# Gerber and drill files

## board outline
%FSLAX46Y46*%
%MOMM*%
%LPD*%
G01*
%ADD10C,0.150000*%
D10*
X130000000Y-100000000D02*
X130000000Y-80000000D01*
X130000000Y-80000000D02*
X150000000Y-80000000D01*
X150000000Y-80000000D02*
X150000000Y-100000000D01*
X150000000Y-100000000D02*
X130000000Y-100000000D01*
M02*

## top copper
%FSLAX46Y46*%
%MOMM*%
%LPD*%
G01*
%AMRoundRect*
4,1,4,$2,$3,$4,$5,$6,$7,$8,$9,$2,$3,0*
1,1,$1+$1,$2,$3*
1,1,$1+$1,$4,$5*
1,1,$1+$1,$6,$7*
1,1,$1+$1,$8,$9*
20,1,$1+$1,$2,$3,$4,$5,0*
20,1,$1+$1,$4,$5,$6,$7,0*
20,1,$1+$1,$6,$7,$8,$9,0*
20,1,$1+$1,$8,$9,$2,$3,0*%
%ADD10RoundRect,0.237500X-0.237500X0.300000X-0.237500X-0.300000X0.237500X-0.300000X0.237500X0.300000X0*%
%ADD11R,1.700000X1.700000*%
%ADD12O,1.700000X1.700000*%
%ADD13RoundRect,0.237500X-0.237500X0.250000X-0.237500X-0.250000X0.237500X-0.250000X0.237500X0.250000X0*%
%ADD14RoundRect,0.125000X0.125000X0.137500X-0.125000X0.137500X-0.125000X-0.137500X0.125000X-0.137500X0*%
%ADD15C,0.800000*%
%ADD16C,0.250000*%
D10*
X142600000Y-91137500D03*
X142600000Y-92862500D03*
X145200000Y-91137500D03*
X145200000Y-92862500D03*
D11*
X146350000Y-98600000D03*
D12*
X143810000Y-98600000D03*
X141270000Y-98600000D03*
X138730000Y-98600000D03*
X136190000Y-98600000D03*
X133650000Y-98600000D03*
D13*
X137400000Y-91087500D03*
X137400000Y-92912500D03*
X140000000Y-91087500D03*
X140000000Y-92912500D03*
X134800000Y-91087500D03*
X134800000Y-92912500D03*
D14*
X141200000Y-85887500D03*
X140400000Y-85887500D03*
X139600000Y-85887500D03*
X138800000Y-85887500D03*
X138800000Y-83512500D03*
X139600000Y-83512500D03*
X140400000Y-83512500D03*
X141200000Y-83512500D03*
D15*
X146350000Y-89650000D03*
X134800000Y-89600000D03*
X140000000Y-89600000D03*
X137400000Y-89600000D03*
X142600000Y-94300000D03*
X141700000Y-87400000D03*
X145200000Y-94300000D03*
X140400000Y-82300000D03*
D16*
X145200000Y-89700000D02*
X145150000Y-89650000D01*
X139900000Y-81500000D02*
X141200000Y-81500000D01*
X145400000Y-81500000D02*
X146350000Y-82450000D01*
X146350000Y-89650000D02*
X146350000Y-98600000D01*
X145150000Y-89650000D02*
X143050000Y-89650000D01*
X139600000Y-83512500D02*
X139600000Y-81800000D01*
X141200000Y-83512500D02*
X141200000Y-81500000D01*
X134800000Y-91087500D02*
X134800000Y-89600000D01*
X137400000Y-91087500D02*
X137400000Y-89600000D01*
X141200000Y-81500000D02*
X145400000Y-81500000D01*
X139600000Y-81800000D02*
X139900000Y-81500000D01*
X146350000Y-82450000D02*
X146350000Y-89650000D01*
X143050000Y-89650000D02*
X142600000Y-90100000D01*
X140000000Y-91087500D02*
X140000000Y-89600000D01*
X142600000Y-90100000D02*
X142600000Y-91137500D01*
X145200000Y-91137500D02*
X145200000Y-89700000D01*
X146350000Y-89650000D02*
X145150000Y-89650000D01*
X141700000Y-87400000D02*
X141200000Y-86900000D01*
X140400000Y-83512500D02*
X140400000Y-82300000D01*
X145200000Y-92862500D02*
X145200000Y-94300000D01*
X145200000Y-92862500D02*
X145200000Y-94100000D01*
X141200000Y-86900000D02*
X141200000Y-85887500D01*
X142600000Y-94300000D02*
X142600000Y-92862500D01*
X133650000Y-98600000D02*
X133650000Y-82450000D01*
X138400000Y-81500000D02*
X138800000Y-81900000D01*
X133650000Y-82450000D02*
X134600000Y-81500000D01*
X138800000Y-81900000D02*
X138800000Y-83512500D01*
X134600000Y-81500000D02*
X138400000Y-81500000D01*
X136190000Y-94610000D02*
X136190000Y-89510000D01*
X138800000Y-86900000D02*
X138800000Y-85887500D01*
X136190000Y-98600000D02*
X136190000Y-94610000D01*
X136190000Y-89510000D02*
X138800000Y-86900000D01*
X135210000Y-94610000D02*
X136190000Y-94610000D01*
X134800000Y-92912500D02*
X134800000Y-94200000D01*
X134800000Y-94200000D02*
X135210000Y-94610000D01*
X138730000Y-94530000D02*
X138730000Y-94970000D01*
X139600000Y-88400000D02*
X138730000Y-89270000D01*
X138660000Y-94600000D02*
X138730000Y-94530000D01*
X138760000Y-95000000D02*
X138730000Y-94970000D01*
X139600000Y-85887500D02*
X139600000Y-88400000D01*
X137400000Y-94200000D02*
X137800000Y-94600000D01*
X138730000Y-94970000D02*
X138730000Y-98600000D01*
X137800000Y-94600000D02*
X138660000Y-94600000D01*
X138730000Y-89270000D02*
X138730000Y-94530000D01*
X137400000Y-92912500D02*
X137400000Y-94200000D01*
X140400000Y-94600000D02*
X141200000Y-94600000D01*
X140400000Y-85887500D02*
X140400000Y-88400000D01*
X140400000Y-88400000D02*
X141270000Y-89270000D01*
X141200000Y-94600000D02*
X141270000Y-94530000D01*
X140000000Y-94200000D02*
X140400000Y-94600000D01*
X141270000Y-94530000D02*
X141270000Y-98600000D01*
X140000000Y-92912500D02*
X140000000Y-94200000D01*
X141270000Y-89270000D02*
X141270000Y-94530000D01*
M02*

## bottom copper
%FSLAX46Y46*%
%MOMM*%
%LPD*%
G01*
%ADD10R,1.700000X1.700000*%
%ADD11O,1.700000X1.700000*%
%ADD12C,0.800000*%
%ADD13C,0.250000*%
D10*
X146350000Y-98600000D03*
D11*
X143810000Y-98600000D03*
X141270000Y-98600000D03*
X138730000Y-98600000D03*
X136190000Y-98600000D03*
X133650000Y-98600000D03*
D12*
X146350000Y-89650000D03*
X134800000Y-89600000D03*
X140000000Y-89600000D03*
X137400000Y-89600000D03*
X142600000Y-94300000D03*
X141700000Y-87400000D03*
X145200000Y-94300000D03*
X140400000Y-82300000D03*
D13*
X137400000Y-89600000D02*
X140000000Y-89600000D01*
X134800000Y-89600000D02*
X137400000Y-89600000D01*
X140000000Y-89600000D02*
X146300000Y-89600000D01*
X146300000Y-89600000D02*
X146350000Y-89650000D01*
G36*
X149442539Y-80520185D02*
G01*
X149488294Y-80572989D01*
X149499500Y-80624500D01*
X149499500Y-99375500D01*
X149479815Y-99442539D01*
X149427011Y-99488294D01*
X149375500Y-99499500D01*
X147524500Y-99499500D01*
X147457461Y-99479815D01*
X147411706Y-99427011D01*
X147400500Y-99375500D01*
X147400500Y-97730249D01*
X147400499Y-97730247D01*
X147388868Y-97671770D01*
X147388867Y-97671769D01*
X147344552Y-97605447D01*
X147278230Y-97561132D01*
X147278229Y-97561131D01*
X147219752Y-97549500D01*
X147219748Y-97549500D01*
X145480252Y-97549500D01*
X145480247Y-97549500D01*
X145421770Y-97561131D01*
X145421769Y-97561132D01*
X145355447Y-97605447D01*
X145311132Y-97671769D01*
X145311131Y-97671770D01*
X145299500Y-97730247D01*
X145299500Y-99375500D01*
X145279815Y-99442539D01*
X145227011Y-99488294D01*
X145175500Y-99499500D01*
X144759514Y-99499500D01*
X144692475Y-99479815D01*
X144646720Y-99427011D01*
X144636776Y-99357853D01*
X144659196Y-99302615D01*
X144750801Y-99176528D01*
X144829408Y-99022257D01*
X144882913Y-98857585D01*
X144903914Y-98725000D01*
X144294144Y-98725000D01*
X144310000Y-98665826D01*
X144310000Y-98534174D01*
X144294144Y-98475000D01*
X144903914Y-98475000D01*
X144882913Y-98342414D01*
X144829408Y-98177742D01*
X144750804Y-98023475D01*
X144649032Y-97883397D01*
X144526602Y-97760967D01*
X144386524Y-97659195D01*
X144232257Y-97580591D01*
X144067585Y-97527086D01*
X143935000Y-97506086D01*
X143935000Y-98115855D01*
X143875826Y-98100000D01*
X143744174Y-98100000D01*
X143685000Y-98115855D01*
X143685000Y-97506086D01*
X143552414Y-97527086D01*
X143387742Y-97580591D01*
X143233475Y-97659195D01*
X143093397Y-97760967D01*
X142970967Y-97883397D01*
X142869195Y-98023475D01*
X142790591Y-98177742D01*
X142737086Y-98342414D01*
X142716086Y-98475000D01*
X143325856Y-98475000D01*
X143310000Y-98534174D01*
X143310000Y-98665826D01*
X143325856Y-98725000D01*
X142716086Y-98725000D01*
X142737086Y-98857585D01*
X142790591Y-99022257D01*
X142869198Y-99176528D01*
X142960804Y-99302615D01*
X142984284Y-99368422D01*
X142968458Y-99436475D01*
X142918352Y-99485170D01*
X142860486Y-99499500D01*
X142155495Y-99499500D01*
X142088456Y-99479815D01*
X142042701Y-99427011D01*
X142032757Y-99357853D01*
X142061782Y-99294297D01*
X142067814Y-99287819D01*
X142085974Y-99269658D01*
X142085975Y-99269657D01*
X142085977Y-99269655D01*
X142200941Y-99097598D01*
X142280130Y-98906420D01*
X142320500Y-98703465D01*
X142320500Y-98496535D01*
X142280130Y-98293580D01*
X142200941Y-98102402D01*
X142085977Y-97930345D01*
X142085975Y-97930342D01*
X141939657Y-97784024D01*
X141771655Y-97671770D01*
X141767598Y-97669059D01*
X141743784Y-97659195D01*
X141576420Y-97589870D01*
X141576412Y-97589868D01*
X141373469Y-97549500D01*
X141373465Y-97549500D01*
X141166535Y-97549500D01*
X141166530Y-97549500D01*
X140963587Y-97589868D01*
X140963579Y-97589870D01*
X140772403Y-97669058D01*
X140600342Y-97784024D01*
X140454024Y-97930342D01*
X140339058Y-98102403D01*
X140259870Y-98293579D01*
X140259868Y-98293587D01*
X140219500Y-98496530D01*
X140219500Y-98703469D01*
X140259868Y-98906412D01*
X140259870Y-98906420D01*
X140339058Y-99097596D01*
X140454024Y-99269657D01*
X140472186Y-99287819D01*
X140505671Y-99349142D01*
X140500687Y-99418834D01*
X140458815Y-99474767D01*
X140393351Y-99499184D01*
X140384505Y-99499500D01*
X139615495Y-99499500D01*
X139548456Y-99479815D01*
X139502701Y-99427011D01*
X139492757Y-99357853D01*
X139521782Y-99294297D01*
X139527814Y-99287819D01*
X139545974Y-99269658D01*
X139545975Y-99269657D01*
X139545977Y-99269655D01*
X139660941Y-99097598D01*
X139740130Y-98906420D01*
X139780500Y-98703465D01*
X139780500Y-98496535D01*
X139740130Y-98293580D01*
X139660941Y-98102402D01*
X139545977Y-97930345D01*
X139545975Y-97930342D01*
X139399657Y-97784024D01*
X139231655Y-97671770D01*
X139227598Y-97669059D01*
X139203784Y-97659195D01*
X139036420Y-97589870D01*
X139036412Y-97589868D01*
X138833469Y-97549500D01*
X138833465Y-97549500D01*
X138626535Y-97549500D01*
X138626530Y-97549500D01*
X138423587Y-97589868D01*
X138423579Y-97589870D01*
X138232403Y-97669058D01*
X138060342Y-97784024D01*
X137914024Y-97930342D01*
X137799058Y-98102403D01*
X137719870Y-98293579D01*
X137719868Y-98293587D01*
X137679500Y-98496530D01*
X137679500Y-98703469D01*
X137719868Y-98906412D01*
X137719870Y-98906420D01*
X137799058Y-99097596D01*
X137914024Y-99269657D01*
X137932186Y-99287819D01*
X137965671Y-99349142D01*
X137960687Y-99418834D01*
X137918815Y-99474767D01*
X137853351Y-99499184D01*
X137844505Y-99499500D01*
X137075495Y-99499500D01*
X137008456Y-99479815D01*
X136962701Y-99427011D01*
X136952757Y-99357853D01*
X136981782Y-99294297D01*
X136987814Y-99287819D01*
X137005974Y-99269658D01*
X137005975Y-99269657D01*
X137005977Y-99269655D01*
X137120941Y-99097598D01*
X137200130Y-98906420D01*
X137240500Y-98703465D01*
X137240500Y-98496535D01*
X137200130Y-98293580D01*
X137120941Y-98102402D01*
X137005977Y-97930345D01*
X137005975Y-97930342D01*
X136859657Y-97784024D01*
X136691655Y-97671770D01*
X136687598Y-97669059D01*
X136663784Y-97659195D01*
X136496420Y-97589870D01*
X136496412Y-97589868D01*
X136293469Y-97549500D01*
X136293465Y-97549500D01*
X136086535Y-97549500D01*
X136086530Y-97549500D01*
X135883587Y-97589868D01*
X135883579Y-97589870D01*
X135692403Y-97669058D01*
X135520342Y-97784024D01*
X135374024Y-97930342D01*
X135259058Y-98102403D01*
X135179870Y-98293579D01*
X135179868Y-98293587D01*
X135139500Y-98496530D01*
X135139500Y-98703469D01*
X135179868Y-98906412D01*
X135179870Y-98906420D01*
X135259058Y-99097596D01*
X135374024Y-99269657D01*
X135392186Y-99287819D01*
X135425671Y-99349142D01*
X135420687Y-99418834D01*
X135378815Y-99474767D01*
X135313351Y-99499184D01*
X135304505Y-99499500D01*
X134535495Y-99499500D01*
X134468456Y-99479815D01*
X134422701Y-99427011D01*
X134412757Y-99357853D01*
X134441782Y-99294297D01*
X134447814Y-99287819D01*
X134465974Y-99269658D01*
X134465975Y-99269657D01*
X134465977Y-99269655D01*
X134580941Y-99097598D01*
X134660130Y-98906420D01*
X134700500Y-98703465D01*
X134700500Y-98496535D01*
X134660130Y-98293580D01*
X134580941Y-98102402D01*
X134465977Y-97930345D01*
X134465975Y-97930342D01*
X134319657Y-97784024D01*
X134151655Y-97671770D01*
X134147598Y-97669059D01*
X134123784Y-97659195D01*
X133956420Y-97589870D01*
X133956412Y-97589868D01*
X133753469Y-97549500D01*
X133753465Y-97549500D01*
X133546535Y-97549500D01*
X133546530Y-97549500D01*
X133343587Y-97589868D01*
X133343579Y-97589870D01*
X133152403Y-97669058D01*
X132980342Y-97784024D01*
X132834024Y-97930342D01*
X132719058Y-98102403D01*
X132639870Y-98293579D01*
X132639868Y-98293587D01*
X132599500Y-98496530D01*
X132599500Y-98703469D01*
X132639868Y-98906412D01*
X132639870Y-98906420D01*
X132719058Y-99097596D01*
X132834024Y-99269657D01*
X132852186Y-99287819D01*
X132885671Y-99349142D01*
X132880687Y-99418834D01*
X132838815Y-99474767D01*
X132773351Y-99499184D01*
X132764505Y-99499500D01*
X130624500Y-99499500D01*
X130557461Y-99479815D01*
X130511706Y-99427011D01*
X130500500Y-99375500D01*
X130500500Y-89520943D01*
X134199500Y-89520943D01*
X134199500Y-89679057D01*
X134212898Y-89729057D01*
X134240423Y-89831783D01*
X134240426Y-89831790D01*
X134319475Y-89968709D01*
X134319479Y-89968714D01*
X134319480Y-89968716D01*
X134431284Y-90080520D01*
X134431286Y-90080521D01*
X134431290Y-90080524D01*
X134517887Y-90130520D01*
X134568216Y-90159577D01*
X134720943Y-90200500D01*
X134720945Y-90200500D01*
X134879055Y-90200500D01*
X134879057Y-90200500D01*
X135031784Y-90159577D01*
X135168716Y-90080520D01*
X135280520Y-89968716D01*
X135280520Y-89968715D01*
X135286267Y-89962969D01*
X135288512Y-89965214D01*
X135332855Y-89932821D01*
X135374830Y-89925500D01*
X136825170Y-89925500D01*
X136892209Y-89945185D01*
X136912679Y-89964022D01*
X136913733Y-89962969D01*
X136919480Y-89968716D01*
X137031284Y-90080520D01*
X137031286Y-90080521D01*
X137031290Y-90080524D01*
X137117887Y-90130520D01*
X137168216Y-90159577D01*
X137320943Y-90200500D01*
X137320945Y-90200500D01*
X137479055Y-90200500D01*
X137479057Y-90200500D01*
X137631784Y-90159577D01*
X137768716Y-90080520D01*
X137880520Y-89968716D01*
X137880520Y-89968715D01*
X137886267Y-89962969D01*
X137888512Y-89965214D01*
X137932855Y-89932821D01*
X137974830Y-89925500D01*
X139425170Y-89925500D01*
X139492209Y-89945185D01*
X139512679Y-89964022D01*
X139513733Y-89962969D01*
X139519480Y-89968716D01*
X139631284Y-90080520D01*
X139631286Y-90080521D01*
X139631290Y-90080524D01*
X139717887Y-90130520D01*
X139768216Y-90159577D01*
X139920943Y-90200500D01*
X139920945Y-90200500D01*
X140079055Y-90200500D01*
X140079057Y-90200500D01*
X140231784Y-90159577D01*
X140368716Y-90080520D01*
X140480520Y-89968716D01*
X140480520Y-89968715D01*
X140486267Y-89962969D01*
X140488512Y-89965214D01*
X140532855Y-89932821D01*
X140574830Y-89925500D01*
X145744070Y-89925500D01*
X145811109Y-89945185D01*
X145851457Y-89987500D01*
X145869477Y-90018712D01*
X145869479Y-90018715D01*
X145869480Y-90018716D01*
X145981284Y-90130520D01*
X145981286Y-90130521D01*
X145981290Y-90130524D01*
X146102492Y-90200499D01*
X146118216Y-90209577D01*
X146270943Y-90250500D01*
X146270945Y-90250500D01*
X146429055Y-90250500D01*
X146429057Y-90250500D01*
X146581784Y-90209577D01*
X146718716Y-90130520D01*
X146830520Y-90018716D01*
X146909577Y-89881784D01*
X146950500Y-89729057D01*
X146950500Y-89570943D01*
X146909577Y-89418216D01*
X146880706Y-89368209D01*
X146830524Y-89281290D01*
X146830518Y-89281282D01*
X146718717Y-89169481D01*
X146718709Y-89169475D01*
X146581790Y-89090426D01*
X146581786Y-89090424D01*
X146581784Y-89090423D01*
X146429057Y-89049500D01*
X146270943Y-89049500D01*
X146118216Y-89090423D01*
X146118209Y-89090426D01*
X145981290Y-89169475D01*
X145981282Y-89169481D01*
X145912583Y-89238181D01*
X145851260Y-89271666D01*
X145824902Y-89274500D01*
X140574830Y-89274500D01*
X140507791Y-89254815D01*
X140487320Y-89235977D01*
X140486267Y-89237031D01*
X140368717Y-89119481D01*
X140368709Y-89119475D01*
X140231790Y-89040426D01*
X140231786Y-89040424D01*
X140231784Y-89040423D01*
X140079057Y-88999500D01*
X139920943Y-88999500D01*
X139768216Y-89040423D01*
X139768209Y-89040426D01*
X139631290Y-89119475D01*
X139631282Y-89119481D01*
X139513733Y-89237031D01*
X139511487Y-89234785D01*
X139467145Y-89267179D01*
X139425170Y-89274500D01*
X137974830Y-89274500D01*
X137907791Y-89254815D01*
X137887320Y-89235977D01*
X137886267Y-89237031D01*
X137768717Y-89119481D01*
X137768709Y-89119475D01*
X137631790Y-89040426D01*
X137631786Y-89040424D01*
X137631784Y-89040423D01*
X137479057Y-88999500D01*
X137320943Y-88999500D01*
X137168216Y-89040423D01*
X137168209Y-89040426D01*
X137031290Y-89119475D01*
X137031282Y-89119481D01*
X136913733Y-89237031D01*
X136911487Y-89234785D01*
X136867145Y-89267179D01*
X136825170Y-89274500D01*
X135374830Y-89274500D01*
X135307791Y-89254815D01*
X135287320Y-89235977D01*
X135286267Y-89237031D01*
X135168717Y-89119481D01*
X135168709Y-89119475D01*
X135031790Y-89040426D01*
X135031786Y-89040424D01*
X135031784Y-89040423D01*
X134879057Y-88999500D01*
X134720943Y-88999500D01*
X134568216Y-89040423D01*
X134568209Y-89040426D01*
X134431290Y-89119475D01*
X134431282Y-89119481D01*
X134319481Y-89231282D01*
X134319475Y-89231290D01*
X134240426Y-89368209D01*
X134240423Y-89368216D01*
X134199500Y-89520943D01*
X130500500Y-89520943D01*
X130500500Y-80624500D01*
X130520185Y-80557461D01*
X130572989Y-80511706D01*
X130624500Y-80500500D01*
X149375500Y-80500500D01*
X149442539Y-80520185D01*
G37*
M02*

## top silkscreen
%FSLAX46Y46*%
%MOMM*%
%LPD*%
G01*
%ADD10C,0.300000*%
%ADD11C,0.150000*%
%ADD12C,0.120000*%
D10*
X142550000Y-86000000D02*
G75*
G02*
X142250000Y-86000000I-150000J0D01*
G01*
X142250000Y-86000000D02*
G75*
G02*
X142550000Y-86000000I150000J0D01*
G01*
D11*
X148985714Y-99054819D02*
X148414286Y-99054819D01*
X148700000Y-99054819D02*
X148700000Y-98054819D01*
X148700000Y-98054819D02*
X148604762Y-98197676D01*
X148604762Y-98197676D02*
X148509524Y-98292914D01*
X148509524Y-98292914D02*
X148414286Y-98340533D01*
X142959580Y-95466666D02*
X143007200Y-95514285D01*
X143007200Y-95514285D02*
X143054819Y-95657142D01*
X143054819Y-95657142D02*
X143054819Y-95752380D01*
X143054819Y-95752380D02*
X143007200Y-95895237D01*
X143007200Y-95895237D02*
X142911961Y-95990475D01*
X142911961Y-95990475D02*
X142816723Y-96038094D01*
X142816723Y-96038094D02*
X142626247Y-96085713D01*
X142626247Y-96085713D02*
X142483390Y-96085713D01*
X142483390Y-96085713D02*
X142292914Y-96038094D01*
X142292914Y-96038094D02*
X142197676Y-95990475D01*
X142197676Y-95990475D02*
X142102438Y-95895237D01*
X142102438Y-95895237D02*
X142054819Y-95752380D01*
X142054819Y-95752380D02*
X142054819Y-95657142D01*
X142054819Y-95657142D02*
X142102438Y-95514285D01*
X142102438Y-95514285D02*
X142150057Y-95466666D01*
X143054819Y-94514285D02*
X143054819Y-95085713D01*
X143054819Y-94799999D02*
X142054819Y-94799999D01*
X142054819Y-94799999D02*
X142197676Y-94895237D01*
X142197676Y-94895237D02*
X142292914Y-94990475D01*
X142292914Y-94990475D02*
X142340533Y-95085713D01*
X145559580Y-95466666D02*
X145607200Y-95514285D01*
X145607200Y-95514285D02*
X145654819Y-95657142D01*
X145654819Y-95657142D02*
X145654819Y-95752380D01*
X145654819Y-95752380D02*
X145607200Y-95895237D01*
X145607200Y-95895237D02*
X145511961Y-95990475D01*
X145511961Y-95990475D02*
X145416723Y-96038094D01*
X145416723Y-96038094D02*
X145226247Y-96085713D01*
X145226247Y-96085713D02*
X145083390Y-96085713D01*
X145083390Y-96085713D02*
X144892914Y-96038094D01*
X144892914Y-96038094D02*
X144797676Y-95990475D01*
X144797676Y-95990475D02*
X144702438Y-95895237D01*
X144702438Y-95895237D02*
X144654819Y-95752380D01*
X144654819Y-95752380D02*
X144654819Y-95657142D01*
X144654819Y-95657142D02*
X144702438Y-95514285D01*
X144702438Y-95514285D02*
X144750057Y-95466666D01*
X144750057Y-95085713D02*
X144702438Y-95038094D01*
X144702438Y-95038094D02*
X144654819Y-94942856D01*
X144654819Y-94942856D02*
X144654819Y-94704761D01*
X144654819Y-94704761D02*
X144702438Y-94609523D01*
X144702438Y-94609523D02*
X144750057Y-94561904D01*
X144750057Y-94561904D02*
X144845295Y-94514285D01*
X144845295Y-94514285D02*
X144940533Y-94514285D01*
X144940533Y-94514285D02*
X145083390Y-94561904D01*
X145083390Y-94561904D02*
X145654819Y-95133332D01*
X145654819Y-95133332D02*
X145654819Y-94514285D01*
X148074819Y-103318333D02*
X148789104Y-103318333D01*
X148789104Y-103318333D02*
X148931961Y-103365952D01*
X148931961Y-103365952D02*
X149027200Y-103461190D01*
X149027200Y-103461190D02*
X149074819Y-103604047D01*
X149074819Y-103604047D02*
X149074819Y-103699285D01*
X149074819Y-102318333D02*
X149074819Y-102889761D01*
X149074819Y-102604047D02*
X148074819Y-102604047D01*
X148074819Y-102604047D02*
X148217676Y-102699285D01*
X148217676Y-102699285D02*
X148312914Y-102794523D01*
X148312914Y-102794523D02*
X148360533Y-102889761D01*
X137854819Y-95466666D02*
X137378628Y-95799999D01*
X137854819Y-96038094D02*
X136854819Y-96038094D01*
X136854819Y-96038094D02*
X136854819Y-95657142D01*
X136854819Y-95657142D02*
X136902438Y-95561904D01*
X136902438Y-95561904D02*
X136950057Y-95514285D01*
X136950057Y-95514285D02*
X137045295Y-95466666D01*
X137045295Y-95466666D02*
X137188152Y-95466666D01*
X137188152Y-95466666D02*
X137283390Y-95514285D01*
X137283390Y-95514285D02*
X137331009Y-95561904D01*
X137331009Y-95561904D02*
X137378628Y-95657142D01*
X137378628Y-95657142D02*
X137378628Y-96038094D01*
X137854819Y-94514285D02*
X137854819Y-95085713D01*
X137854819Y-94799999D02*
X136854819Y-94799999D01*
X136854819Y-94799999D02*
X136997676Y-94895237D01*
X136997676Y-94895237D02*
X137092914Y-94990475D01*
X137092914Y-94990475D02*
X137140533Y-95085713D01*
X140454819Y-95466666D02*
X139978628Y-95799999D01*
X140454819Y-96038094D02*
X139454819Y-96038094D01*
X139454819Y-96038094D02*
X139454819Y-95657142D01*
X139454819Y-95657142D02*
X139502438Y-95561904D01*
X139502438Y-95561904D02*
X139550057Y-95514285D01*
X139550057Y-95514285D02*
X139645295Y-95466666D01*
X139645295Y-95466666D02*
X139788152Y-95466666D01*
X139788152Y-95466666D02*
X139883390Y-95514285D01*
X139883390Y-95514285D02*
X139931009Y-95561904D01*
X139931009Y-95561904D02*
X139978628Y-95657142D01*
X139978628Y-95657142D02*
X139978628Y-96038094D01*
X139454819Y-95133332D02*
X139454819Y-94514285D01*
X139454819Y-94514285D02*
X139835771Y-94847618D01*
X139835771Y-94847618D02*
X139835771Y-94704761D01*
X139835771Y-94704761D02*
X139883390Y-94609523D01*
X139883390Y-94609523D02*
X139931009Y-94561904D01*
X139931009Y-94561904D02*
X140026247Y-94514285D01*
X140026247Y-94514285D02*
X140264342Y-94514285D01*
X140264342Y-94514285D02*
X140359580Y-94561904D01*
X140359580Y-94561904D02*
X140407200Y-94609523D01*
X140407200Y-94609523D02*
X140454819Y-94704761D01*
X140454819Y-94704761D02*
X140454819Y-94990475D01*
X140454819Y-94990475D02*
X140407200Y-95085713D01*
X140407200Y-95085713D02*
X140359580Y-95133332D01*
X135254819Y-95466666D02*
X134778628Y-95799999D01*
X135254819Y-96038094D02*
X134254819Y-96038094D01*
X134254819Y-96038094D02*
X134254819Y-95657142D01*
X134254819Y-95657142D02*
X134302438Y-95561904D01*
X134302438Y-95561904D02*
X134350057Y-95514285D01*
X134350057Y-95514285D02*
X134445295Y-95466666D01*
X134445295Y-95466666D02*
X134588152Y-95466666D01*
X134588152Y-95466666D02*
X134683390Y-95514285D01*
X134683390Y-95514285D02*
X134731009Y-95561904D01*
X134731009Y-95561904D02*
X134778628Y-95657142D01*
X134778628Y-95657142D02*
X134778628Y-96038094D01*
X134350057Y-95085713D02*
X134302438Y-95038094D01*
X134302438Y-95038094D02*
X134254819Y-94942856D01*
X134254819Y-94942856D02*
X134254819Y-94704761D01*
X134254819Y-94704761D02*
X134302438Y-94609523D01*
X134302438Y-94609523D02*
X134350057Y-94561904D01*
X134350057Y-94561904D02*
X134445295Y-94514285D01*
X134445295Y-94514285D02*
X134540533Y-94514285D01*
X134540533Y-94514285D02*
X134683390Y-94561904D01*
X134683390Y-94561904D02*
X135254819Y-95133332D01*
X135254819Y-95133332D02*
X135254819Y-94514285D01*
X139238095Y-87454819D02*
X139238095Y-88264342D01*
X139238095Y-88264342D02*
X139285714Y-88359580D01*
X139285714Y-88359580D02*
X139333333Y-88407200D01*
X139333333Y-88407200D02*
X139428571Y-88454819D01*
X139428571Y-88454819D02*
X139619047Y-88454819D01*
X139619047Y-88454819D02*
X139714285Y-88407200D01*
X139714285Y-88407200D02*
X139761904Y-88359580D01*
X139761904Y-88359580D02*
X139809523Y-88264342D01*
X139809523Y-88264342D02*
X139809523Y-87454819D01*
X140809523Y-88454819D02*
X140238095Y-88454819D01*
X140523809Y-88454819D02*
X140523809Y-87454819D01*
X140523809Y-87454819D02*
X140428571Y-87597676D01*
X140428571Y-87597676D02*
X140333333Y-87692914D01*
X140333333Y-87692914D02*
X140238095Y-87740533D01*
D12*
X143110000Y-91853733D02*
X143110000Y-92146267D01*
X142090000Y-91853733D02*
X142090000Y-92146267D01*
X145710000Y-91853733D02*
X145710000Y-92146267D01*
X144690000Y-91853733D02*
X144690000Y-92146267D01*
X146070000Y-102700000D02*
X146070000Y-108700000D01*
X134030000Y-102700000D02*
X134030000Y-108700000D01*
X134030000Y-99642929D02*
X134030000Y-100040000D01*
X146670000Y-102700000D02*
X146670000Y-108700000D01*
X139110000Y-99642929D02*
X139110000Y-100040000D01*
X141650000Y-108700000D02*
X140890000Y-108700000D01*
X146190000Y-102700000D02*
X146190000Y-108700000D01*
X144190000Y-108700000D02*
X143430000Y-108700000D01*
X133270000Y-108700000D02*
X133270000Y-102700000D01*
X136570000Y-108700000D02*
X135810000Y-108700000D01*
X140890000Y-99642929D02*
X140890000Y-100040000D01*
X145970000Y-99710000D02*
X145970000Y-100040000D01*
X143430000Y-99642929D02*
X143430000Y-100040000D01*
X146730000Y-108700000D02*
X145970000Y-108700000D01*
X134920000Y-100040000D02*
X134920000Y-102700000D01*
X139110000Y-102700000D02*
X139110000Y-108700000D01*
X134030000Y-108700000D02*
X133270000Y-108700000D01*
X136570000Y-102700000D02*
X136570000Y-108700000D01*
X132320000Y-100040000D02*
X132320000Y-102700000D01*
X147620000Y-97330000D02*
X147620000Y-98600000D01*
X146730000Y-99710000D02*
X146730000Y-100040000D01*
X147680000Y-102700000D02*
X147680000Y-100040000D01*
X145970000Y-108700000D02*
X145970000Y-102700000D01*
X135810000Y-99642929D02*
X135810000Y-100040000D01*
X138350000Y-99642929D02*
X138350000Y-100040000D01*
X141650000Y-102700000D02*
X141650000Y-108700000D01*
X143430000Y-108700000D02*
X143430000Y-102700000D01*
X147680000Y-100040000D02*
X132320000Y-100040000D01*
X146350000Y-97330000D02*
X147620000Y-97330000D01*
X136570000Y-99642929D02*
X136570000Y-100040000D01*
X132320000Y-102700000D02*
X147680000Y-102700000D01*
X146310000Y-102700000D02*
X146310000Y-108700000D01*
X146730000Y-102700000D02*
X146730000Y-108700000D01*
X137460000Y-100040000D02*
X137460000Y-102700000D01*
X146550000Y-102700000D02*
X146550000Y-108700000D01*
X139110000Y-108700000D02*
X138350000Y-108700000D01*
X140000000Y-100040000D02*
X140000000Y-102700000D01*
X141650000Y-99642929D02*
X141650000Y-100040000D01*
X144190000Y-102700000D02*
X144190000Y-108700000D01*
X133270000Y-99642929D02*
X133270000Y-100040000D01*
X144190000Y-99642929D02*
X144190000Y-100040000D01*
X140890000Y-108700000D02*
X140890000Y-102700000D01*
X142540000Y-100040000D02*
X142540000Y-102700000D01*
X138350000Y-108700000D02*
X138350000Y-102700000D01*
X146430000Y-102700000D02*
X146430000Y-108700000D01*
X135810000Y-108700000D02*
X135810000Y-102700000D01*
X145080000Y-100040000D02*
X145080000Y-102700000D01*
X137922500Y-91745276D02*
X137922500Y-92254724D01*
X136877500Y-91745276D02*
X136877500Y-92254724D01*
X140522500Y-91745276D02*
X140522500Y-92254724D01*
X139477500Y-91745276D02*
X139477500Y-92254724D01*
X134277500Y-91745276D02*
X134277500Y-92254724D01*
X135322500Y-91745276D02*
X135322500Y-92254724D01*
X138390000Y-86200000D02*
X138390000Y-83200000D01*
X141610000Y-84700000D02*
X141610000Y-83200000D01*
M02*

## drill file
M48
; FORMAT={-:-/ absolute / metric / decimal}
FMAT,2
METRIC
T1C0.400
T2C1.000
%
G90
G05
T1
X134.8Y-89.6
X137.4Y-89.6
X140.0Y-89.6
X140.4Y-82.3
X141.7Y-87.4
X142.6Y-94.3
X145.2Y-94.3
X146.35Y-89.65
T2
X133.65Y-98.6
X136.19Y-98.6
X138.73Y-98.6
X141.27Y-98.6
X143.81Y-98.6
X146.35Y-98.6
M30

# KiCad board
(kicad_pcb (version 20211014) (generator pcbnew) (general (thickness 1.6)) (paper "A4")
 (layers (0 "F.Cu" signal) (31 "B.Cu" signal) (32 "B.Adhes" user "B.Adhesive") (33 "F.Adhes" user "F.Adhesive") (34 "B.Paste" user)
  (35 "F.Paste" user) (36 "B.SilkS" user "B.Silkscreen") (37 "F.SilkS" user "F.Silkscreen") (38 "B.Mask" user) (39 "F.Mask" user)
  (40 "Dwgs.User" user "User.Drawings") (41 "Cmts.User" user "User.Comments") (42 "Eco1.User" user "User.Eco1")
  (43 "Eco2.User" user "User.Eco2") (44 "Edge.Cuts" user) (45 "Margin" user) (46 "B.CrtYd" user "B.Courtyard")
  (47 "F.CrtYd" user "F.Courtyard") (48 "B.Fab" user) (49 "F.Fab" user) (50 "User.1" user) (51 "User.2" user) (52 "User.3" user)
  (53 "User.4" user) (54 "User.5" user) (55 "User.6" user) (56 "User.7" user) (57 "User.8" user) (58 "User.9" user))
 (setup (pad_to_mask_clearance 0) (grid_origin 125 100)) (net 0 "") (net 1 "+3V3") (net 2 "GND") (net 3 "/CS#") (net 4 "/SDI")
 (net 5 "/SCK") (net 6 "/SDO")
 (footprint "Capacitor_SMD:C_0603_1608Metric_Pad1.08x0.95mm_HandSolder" (layer "F.Cu") (at 142.6 92 -90)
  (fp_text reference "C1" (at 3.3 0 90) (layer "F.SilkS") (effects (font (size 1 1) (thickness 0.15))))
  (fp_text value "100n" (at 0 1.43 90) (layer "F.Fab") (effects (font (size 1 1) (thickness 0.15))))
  (fp_line (start -0.146267 -0.51) (end 0.146267 -0.51) (layer "F.SilkS") (width 0.12))
  (fp_line (start -0.146267 0.51) (end 0.146267 0.51) (layer "F.SilkS") (width 0.12))
  (pad "1" smd roundrect (at -0.8625 0 270) (size 1.075 0.95) (layers "F.Cu" "F.Paste" "F.Mask") (roundrect_rratio 0.25) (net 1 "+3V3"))
  (pad "2" smd roundrect (at 0.8625 0 270) (size 1.075 0.95) (layers "F.Cu" "F.Paste" "F.Mask") (roundrect_rratio 0.25) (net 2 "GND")))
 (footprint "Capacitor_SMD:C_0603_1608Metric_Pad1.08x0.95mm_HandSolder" (layer "F.Cu") (at 145.2 92 -90)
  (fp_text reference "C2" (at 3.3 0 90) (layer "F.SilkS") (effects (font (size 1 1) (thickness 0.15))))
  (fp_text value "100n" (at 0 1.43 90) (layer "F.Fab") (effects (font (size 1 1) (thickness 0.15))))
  (fp_line (start -0.146267 -0.51) (end 0.146267 -0.51) (layer "F.SilkS") (width 0.12))
  (fp_line (start -0.146267 0.51) (end 0.146267 0.51) (layer "F.SilkS") (width 0.12))
  (pad "1" smd roundrect (at -0.8625 0 270) (size 1.075 0.95) (layers "F.Cu" "F.Paste" "F.Mask") (roundrect_rratio 0.25) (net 1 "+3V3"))
  (pad "2" smd roundrect (at 0.8625 0 270) (size 1.075 0.95) (layers "F.Cu" "F.Paste" "F.Mask") (roundrect_rratio 0.25) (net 2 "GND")))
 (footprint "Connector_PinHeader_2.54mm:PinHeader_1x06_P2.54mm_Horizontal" (layer "F.Cu") (at 146.35 98.6 -90)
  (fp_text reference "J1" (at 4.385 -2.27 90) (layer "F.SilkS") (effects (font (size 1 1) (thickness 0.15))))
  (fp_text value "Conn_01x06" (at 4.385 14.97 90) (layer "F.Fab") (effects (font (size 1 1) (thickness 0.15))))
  (fp_line (start 4.1 0.28) (end 10.1 0.28) (layer "F.SilkS") (width 0.12))
  (fp_line (start 4.1 12.32) (end 10.1 12.32) (layer "F.SilkS") (width 0.12))
  (fp_line (start 1.042929 12.32) (end 1.44 12.32) (layer "F.SilkS") (width 0.12))
  (fp_line (start 4.1 -0.32) (end 10.1 -0.32) (layer "F.SilkS") (width 0.12))
  (fp_line (start 1.042929 7.24) (end 1.44 7.24) (layer "F.SilkS") (width 0.12))
  (fp_line (start 10.1 4.7) (end 10.1 5.46) (layer "F.SilkS") (width 0.12))
  (fp_line (start 4.1 0.16) (end 10.1 0.16) (layer "F.SilkS") (width 0.12))
  (fp_line (start 10.1 2.16) (end 10.1 2.92) (layer "F.SilkS") (width 0.12))
  (fp_line (start 10.1 13.08) (end 4.1 13.08) (layer "F.SilkS") (width 0.12))
  (fp_line (start 10.1 9.78) (end 10.1 10.54) (layer "F.SilkS") (width 0.12))
  (fp_line (start 1.042929 5.46) (end 1.44 5.46) (layer "F.SilkS") (width 0.12))
  (fp_line (start 1.11 0.38) (end 1.44 0.38) (layer "F.SilkS") (width 0.12))
  (fp_line (start 1.042929 2.92) (end 1.44 2.92) (layer "F.SilkS") (width 0.12))
  (fp_line (start 10.1 -0.38) (end 10.1 0.38) (layer "F.SilkS") (width 0.12))
  (fp_line (start 1.44 11.43) (end 4.1 11.43) (layer "F.SilkS") (width 0.12))
  (fp_line (start 4.1 7.24) (end 10.1 7.24) (layer "F.SilkS") (width 0.12))
  (fp_line (start 10.1 12.32) (end 10.1 13.08) (layer "F.SilkS") (width 0.12))
  (fp_line (start 4.1 9.78) (end 10.1 9.78) (layer "F.SilkS") (width 0.12))
  (fp_line (start 1.44 14.03) (end 4.1 14.03) (layer "F.SilkS") (width 0.12))
  (fp_line (start -1.27 -1.27) (end 0 -1.27) (layer "F.SilkS") (width 0.12))
  (fp_line (start 1.11 -0.38) (end 1.44 -0.38) (layer "F.SilkS") (width 0.12))
  (fp_line (start 4.1 -1.33) (end 1.44 -1.33) (layer "F.SilkS") (width 0.12))
  (fp_line (start 10.1 0.38) (end 4.1 0.38) (layer "F.SilkS") (width 0.12))
  (fp_line (start 1.042929 10.54) (end 1.44 10.54) (layer "F.SilkS") (width 0.12))
  (fp_line (start 1.042929 8) (end 1.44 8) (layer "F.SilkS") (width 0.12))
  (fp_line (start 4.1 4.7) (end 10.1 4.7) (layer "F.SilkS") (width 0.12))
  (fp_line (start 10.1 2.92) (end 4.1 2.92) (layer "F.SilkS") (width 0.12))
  (fp_line (start 1.44 -1.33) (end 1.44 14.03) (layer "F.SilkS") (width 0.12))
  (fp_line (start -1.27 0) (end -1.27 -1.27) (layer "F.SilkS") (width 0.12))
  (fp_line (start 1.042929 9.78) (end 1.44 9.78) (layer "F.SilkS") (width 0.12))
  (fp_line (start 4.1 14.03) (end 4.1 -1.33) (layer "F.SilkS") (width 0.12))
  (fp_line (start 4.1 0.04) (end 10.1 0.04) (layer "F.SilkS") (width 0.12))
  (fp_line (start 4.1 -0.38) (end 10.1 -0.38) (layer "F.SilkS") (width 0.12))
  (fp_line (start 1.44 8.89) (end 4.1 8.89) (layer "F.SilkS") (width 0.12))
  (fp_line (start 4.1 -0.2) (end 10.1 -0.2) (layer "F.SilkS") (width 0.12))
  (fp_line (start 10.1 7.24) (end 10.1 8) (layer "F.SilkS") (width 0.12))
  (fp_line (start 1.44 6.35) (end 4.1 6.35) (layer "F.SilkS") (width 0.12))
  (fp_line (start 1.042929 4.7) (end 1.44 4.7) (layer "F.SilkS") (width 0.12))
  (fp_line (start 4.1 2.16) (end 10.1 2.16) (layer "F.SilkS") (width 0.12))
  (fp_line (start 1.042929 13.08) (end 1.44 13.08) (layer "F.SilkS") (width 0.12))
  (fp_line (start 1.042929 2.16) (end 1.44 2.16) (layer "F.SilkS") (width 0.12))
  (fp_line (start 10.1 5.46) (end 4.1 5.46) (layer "F.SilkS") (width 0.12))
  (fp_line (start 1.44 3.81) (end 4.1 3.81) (layer "F.SilkS") (width 0.12))
  (fp_line (start 10.1 8) (end 4.1 8) (layer "F.SilkS") (width 0.12))
  (fp_line (start 4.1 -0.08) (end 10.1 -0.08) (layer "F.SilkS") (width 0.12))
  (fp_line (start 10.1 10.54) (end 4.1 10.54) (layer "F.SilkS") (width 0.12))
  (fp_line (start 1.44 1.27) (end 4.1 1.27) (layer "F.SilkS") (width 0.12))
  (pad "1" thru_hole rect (at 0 0 270) (size 1.7 1.7) (drill 1) (layers *.Cu *.Mask) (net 1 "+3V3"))
  (pad "2" thru_hole oval (at 0 2.54 270) (size 1.7 1.7) (drill 1) (layers *.Cu *.Mask) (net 2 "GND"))
  (pad "3" thru_hole oval (at 0 5.08 270) (size 1.7 1.7) (drill 1) (layers *.Cu *.Mask) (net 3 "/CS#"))
  (pad "4" thru_hole oval (at 0 7.62 270) (size 1.7 1.7) (drill 1) (layers *.Cu *.Mask) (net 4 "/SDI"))
  (pad "5" thru_hole oval (at 0 10.16 270) (size 1.7 1.7) (drill 1) (layers *.Cu *.Mask) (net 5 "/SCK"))
  (pad "6" thru_hole oval (at 0 12.7 270) (size 1.7 1.7) (drill 1) (layers *.Cu *.Mask) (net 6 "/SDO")))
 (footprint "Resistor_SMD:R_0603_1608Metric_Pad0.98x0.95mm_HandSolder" (layer "F.Cu") (at 137.4 92 -90)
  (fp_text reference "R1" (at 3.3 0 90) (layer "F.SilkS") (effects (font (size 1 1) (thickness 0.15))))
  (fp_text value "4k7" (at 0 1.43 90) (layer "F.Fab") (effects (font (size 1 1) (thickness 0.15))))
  (fp_line (start -0.254724 -0.5225) (end 0.254724 -0.5225) (layer "F.SilkS") (width 0.12))
  (fp_line (start -0.254724 0.5225) (end 0.254724 0.5225) (layer "F.SilkS") (width 0.12))
  (pad "1" smd roundrect (at -0.9125 0 270) (size 0.975 0.95) (layers "F.Cu" "F.Paste" "F.Mask") (roundrect_rratio 0.25) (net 1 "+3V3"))
  (pad "2" smd roundrect (at 0.9125 0 270) (size 0.975 0.95) (layers "F.Cu" "F.Paste" "F.Mask") (roundrect_rratio 0.25) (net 4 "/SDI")))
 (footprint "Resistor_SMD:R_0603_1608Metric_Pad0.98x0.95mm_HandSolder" (layer "F.Cu") (at 140 92 -90)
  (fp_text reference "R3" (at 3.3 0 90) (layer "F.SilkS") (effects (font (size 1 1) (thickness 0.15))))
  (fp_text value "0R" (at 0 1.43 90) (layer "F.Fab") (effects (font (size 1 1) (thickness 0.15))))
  (fp_line (start -0.254724 -0.5225) (end 0.254724 -0.5225) (layer "F.SilkS") (width 0.12))
  (fp_line (start -0.254724 0.5225) (end 0.254724 0.5225) (layer "F.SilkS") (width 0.12))
  (pad "1" smd roundrect (at -0.9125 0 270) (size 0.975 0.95) (layers "F.Cu" "F.Paste" "F.Mask") (roundrect_rratio 0.25) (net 1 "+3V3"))
  (pad "2" smd roundrect (at 0.9125 0 270) (size 0.975 0.95) (layers "F.Cu" "F.Paste" "F.Mask") (roundrect_rratio 0.25) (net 3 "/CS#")))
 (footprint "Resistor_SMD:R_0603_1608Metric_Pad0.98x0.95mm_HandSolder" (layer "F.Cu") (at 134.8 92 -90)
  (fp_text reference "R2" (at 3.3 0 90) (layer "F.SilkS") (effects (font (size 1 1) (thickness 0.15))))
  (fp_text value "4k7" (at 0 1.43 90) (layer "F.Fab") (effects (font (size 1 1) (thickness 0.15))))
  (fp_line (start -0.254724 0.5225) (end 0.254724 0.5225) (layer "F.SilkS") (width 0.12))
  (fp_line (start -0.254724 -0.5225) (end 0.254724 -0.5225) (layer "F.SilkS") (width 0.12))
  (pad "1" smd roundrect (at -0.9125 0 270) (size 0.975 0.95) (layers "F.Cu" "F.Paste" "F.Mask") (roundrect_rratio 0.25) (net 1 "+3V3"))
  (pad "2" smd roundrect (at 0.9125 0 270) (size 0.975 0.95) (layers "F.Cu" "F.Paste" "F.Mask") (roundrect_rratio 0.25) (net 5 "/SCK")))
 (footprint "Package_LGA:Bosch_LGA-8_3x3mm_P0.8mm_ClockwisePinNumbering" (layer "F.Cu") (at 140 84.7 180)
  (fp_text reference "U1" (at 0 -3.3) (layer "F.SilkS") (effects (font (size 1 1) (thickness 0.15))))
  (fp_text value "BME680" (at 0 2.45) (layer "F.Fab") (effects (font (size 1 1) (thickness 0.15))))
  (fp_line (start 1.61 -1.5) (end 1.61 1.5) (layer "F.SilkS") (width 0.12))
  (fp_line (start -1.61 0) (end -1.61 1.5) (layer "F.SilkS") (width 0.12))
  (pad "1" smd roundrect (at -1.2 -1.1875 180) (size 0.5 0.525) (layers "F.Cu" "F.Paste" "F.Mask") (roundrect_rratio 0.25) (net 2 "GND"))
  (pad "2" smd roundrect (at -0.4 -1.1875 180) (size 0.5 0.525) (layers "F.Cu" "F.Paste" "F.Mask") (roundrect_rratio 0.25) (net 3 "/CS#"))
  (pad "3" smd roundrect (at 0.4 -1.1875 180) (size 0.5 0.525) (layers "F.Cu" "F.Paste" "F.Mask") (roundrect_rratio 0.25) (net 4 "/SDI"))
  (pad "4" smd roundrect (at 1.2 -1.1875 180) (size 0.5 0.525) (layers "F.Cu" "F.Paste" "F.Mask") (roundrect_rratio 0.25) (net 5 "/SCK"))
  (pad "5" smd roundrect (at 1.2 1.1875 180) (size 0.5 0.525) (layers "F.Cu" "F.Paste" "F.Mask") (roundrect_rratio 0.25) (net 6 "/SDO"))
  (pad "6" smd roundrect (at 0.4 1.1875 180) (size 0.5 0.525) (layers "F.Cu" "F.Paste" "F.Mask") (roundrect_rratio 0.25) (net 1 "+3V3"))
  (pad "7" smd roundrect (at -0.4 1.1875 180) (size 0.5 0.525) (layers "F.Cu" "F.Paste" "F.Mask") (roundrect_rratio 0.25) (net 2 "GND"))
  (pad "8" smd roundrect (at -1.2 1.1875 180) (size 0.5 0.525) (layers "F.Cu" "F.Paste" "F.Mask") (roundrect_rratio 0.25) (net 1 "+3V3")))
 (gr_circle (center 142.4 86) (end 142.55 86) (layer "F.SilkS") (width 0.3) (fill none))
 (gr_line (start 130 100) (end 130 80) (layer "Edge.Cuts") (width 0.15))
 (gr_line (start 130 80) (end 150 80) (layer "Edge.Cuts") (width 0.15))
 (gr_line (start 150 80) (end 150 100) (layer "Edge.Cuts") (width 0.15))
 (gr_line (start 150 100) (end 130 100) (layer "Edge.Cuts") (width 0.15))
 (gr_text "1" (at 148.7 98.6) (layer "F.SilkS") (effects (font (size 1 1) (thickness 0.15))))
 (segment (start 145.2 89.7) (end 145.15 89.65) (width 0.25) (layer "F.Cu") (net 1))
 (segment (start 139.9 81.5) (end 141.2 81.5) (width 0.25) (layer "F.Cu") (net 1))
 (segment (start 145.4 81.5) (end 146.35 82.45) (width 0.25) (layer "F.Cu") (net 1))
 (segment (start 146.35 89.65) (end 146.35 98.6) (width 0.25) (layer "F.Cu") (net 1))
 (segment (start 145.15 89.65) (end 143.05 89.65) (width 0.25) (layer "F.Cu") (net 1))
 (segment (start 139.6 83.5125) (end 139.6 81.8) (width 0.25) (layer "F.Cu") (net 1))
 (segment (start 141.2 83.5125) (end 141.2 81.5) (width 0.25) (layer "F.Cu") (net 1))
 (segment (start 134.8 91.0875) (end 134.8 89.6) (width 0.25) (layer "F.Cu") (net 1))
 (segment (start 137.4 91.0875) (end 137.4 89.6) (width 0.25) (layer "F.Cu") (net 1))
 (segment (start 141.2 81.5) (end 145.4 81.5) (width 0.25) (layer "F.Cu") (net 1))
 (segment (start 139.6 81.8) (end 139.9 81.5) (width 0.25) (layer "F.Cu") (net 1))
 (segment (start 146.35 82.45) (end 146.35 89.65) (width 0.25) (layer "F.Cu") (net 1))
 (segment (start 143.05 89.65) (end 142.6 90.1) (width 0.25) (layer "F.Cu") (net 1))
 (segment (start 140 91.0875) (end 140 89.6) (width 0.25) (layer "F.Cu") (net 1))
 (segment (start 142.6 90.1) (end 142.6 91.1375) (width 0.25) (layer "F.Cu") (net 1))
 (segment (start 145.2 91.1375) (end 145.2 89.7) (width 0.25) (layer "F.Cu") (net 1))
 (segment (start 146.35 89.65) (end 145.15 89.65) (width 0.25) (layer "F.Cu") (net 1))
 (via (at 146.35 89.65) (size 0.8) (drill 0.4) (layers "F.Cu" "B.Cu") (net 1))
 (via (at 134.8 89.6) (size 0.8) (drill 0.4) (layers "F.Cu" "B.Cu") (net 1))
 (via (at 140 89.6) (size 0.8) (drill 0.4) (layers "F.Cu" "B.Cu") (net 1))
 (via (at 137.4 89.6) (size 0.8) (drill 0.4) (layers "F.Cu" "B.Cu") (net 1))
 (segment (start 137.4 89.6) (end 140 89.6) (width 0.25) (layer "B.Cu") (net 1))
 (segment (start 134.8 89.6) (end 137.4 89.6) (width 0.25) (layer "B.Cu") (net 1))
 (segment (start 140 89.6) (end 146.3 89.6) (width 0.25) (layer "B.Cu") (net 1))
 (segment (start 146.3 89.6) (end 146.35 89.65) (width 0.25) (layer "B.Cu") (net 1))
 (segment (start 141.7 87.4) (end 141.2 86.9) (width 0.25) (layer "F.Cu") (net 2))
 (segment (start 140.4 83.5125) (end 140.4 82.3) (width 0.25) (layer "F.Cu") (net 2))
 (segment (start 145.2 92.8625) (end 145.2 94.3) (width 0.25) (layer "F.Cu") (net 2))
 (segment (start 145.2 92.8625) (end 145.2 94.1) (width 0.25) (layer "F.Cu") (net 2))
 (segment (start 141.2 86.9) (end 141.2 85.8875) (width 0.25) (layer "F.Cu") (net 2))
 (segment (start 142.6 94.3) (end 142.6 92.8625) (width 0.25) (layer "F.Cu") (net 2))
 (via (at 142.6 94.3) (size 0.8) (drill 0.4) (layers "F.Cu" "B.Cu") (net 2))
 (via (at 141.7 87.4) (size 0.8) (drill 0.4) (layers "F.Cu" "B.Cu") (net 2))
 (via (at 145.2 94.3) (size 0.8) (drill 0.4) (layers "F.Cu" "B.Cu") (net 2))
 (via (at 140.4 82.3) (size 0.8) (drill 0.4) (layers "F.Cu" "B.Cu") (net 2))
 (segment (start 133.65 98.6) (end 133.65 82.45) (width 0.25) (layer "F.Cu") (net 6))
 (segment (start 138.4 81.5) (end 138.8 81.9) (width 0.25) (layer "F.Cu") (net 6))
 (segment (start 133.65 82.45) (end 134.6 81.5) (width 0.25) (layer "F.Cu") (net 6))
 (segment (start 138.8 81.9) (end 138.8 83.5125) (width 0.25) (layer "F.Cu") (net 6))
 (segment (start 134.6 81.5) (end 138.4 81.5) (width 0.25) (layer "F.Cu") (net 6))
 (segment (start 136.19 94.61) (end 136.19 89.51) (width 0.25) (layer "F.Cu") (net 5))
 (segment (start 138.8 86.9) (end 138.8 85.8875) (width 0.25) (layer "F.Cu") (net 5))
 (segment (start 136.19 98.6) (end 136.19 94.61) (width 0.25) (layer "F.Cu") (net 5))
 (segment (start 136.19 89.51) (end 138.8 86.9) (width 0.25) (layer "F.Cu") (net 5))
 (segment (start 135.21 94.61) (end 136.19 94.61) (width 0.25) (layer "F.Cu") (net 5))
 (segment (start 134.8 92.9125) (end 134.8 94.2) (width 0.25) (layer "F.Cu") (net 5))
 (segment (start 134.8 94.2) (end 135.21 94.61) (width 0.25) (layer "F.Cu") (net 5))
 (segment (start 138.73 94.53) (end 138.73 94.97) (width 0.25) (layer "F.Cu") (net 4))
 (segment (start 139.6 88.4) (end 138.73 89.27) (width 0.25) (layer "F.Cu") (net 4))
 (segment (start 138.66 94.6) (end 138.73 94.53) (width 0.25) (layer "F.Cu") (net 4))
 (segment (start 138.76 95) (end 138.73 94.97) (width 0.25) (layer "F.Cu") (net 4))
 (segment (start 139.6 85.8875) (end 139.6 88.4) (width 0.25) (layer "F.Cu") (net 4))
 (segment (start 137.4 94.2) (end 137.8 94.6) (width 0.25) (layer "F.Cu") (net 4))
 (segment (start 138.73 94.97) (end 138.73 98.6) (width 0.25) (layer "F.Cu") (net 4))
 (segment (start 137.8 94.6) (end 138.66 94.6) (width 0.25) (layer "F.Cu") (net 4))
 (segment (start 138.73 89.27) (end 138.73 94.53) (width 0.25) (layer "F.Cu") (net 4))
 (segment (start 137.4 92.9125) (end 137.4 94.2) (width 0.25) (layer "F.Cu") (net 4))
 (segment (start 140.4 94.6) (end 141.2 94.6) (width 0.25) (layer "F.Cu") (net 3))
 (segment (start 140.4 85.8875) (end 140.4 88.4) (width 0.25) (layer "F.Cu") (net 3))
 (segment (start 140.4 88.4) (end 141.27 89.27) (width 0.25) (layer "F.Cu") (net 3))
 (segment (start 141.2 94.6) (end 141.27 94.53) (width 0.25) (layer "F.Cu") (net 3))
 (segment (start 140 94.2) (end 140.4 94.6) (width 0.25) (layer "F.Cu") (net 3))
 (segment (start 141.27 94.53) (end 141.27 98.6) (width 0.25) (layer "F.Cu") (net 3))
 (segment (start 140 92.9125) (end 140 94.2) (width 0.25) (layer "F.Cu") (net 3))
 (segment (start 141.27 89.27) (end 141.27 94.53) (width 0.25) (layer "F.Cu") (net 3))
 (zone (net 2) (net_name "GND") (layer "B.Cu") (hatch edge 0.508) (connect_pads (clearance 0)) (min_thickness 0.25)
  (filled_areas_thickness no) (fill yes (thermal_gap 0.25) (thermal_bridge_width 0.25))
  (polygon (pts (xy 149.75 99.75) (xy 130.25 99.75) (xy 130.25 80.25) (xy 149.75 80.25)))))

